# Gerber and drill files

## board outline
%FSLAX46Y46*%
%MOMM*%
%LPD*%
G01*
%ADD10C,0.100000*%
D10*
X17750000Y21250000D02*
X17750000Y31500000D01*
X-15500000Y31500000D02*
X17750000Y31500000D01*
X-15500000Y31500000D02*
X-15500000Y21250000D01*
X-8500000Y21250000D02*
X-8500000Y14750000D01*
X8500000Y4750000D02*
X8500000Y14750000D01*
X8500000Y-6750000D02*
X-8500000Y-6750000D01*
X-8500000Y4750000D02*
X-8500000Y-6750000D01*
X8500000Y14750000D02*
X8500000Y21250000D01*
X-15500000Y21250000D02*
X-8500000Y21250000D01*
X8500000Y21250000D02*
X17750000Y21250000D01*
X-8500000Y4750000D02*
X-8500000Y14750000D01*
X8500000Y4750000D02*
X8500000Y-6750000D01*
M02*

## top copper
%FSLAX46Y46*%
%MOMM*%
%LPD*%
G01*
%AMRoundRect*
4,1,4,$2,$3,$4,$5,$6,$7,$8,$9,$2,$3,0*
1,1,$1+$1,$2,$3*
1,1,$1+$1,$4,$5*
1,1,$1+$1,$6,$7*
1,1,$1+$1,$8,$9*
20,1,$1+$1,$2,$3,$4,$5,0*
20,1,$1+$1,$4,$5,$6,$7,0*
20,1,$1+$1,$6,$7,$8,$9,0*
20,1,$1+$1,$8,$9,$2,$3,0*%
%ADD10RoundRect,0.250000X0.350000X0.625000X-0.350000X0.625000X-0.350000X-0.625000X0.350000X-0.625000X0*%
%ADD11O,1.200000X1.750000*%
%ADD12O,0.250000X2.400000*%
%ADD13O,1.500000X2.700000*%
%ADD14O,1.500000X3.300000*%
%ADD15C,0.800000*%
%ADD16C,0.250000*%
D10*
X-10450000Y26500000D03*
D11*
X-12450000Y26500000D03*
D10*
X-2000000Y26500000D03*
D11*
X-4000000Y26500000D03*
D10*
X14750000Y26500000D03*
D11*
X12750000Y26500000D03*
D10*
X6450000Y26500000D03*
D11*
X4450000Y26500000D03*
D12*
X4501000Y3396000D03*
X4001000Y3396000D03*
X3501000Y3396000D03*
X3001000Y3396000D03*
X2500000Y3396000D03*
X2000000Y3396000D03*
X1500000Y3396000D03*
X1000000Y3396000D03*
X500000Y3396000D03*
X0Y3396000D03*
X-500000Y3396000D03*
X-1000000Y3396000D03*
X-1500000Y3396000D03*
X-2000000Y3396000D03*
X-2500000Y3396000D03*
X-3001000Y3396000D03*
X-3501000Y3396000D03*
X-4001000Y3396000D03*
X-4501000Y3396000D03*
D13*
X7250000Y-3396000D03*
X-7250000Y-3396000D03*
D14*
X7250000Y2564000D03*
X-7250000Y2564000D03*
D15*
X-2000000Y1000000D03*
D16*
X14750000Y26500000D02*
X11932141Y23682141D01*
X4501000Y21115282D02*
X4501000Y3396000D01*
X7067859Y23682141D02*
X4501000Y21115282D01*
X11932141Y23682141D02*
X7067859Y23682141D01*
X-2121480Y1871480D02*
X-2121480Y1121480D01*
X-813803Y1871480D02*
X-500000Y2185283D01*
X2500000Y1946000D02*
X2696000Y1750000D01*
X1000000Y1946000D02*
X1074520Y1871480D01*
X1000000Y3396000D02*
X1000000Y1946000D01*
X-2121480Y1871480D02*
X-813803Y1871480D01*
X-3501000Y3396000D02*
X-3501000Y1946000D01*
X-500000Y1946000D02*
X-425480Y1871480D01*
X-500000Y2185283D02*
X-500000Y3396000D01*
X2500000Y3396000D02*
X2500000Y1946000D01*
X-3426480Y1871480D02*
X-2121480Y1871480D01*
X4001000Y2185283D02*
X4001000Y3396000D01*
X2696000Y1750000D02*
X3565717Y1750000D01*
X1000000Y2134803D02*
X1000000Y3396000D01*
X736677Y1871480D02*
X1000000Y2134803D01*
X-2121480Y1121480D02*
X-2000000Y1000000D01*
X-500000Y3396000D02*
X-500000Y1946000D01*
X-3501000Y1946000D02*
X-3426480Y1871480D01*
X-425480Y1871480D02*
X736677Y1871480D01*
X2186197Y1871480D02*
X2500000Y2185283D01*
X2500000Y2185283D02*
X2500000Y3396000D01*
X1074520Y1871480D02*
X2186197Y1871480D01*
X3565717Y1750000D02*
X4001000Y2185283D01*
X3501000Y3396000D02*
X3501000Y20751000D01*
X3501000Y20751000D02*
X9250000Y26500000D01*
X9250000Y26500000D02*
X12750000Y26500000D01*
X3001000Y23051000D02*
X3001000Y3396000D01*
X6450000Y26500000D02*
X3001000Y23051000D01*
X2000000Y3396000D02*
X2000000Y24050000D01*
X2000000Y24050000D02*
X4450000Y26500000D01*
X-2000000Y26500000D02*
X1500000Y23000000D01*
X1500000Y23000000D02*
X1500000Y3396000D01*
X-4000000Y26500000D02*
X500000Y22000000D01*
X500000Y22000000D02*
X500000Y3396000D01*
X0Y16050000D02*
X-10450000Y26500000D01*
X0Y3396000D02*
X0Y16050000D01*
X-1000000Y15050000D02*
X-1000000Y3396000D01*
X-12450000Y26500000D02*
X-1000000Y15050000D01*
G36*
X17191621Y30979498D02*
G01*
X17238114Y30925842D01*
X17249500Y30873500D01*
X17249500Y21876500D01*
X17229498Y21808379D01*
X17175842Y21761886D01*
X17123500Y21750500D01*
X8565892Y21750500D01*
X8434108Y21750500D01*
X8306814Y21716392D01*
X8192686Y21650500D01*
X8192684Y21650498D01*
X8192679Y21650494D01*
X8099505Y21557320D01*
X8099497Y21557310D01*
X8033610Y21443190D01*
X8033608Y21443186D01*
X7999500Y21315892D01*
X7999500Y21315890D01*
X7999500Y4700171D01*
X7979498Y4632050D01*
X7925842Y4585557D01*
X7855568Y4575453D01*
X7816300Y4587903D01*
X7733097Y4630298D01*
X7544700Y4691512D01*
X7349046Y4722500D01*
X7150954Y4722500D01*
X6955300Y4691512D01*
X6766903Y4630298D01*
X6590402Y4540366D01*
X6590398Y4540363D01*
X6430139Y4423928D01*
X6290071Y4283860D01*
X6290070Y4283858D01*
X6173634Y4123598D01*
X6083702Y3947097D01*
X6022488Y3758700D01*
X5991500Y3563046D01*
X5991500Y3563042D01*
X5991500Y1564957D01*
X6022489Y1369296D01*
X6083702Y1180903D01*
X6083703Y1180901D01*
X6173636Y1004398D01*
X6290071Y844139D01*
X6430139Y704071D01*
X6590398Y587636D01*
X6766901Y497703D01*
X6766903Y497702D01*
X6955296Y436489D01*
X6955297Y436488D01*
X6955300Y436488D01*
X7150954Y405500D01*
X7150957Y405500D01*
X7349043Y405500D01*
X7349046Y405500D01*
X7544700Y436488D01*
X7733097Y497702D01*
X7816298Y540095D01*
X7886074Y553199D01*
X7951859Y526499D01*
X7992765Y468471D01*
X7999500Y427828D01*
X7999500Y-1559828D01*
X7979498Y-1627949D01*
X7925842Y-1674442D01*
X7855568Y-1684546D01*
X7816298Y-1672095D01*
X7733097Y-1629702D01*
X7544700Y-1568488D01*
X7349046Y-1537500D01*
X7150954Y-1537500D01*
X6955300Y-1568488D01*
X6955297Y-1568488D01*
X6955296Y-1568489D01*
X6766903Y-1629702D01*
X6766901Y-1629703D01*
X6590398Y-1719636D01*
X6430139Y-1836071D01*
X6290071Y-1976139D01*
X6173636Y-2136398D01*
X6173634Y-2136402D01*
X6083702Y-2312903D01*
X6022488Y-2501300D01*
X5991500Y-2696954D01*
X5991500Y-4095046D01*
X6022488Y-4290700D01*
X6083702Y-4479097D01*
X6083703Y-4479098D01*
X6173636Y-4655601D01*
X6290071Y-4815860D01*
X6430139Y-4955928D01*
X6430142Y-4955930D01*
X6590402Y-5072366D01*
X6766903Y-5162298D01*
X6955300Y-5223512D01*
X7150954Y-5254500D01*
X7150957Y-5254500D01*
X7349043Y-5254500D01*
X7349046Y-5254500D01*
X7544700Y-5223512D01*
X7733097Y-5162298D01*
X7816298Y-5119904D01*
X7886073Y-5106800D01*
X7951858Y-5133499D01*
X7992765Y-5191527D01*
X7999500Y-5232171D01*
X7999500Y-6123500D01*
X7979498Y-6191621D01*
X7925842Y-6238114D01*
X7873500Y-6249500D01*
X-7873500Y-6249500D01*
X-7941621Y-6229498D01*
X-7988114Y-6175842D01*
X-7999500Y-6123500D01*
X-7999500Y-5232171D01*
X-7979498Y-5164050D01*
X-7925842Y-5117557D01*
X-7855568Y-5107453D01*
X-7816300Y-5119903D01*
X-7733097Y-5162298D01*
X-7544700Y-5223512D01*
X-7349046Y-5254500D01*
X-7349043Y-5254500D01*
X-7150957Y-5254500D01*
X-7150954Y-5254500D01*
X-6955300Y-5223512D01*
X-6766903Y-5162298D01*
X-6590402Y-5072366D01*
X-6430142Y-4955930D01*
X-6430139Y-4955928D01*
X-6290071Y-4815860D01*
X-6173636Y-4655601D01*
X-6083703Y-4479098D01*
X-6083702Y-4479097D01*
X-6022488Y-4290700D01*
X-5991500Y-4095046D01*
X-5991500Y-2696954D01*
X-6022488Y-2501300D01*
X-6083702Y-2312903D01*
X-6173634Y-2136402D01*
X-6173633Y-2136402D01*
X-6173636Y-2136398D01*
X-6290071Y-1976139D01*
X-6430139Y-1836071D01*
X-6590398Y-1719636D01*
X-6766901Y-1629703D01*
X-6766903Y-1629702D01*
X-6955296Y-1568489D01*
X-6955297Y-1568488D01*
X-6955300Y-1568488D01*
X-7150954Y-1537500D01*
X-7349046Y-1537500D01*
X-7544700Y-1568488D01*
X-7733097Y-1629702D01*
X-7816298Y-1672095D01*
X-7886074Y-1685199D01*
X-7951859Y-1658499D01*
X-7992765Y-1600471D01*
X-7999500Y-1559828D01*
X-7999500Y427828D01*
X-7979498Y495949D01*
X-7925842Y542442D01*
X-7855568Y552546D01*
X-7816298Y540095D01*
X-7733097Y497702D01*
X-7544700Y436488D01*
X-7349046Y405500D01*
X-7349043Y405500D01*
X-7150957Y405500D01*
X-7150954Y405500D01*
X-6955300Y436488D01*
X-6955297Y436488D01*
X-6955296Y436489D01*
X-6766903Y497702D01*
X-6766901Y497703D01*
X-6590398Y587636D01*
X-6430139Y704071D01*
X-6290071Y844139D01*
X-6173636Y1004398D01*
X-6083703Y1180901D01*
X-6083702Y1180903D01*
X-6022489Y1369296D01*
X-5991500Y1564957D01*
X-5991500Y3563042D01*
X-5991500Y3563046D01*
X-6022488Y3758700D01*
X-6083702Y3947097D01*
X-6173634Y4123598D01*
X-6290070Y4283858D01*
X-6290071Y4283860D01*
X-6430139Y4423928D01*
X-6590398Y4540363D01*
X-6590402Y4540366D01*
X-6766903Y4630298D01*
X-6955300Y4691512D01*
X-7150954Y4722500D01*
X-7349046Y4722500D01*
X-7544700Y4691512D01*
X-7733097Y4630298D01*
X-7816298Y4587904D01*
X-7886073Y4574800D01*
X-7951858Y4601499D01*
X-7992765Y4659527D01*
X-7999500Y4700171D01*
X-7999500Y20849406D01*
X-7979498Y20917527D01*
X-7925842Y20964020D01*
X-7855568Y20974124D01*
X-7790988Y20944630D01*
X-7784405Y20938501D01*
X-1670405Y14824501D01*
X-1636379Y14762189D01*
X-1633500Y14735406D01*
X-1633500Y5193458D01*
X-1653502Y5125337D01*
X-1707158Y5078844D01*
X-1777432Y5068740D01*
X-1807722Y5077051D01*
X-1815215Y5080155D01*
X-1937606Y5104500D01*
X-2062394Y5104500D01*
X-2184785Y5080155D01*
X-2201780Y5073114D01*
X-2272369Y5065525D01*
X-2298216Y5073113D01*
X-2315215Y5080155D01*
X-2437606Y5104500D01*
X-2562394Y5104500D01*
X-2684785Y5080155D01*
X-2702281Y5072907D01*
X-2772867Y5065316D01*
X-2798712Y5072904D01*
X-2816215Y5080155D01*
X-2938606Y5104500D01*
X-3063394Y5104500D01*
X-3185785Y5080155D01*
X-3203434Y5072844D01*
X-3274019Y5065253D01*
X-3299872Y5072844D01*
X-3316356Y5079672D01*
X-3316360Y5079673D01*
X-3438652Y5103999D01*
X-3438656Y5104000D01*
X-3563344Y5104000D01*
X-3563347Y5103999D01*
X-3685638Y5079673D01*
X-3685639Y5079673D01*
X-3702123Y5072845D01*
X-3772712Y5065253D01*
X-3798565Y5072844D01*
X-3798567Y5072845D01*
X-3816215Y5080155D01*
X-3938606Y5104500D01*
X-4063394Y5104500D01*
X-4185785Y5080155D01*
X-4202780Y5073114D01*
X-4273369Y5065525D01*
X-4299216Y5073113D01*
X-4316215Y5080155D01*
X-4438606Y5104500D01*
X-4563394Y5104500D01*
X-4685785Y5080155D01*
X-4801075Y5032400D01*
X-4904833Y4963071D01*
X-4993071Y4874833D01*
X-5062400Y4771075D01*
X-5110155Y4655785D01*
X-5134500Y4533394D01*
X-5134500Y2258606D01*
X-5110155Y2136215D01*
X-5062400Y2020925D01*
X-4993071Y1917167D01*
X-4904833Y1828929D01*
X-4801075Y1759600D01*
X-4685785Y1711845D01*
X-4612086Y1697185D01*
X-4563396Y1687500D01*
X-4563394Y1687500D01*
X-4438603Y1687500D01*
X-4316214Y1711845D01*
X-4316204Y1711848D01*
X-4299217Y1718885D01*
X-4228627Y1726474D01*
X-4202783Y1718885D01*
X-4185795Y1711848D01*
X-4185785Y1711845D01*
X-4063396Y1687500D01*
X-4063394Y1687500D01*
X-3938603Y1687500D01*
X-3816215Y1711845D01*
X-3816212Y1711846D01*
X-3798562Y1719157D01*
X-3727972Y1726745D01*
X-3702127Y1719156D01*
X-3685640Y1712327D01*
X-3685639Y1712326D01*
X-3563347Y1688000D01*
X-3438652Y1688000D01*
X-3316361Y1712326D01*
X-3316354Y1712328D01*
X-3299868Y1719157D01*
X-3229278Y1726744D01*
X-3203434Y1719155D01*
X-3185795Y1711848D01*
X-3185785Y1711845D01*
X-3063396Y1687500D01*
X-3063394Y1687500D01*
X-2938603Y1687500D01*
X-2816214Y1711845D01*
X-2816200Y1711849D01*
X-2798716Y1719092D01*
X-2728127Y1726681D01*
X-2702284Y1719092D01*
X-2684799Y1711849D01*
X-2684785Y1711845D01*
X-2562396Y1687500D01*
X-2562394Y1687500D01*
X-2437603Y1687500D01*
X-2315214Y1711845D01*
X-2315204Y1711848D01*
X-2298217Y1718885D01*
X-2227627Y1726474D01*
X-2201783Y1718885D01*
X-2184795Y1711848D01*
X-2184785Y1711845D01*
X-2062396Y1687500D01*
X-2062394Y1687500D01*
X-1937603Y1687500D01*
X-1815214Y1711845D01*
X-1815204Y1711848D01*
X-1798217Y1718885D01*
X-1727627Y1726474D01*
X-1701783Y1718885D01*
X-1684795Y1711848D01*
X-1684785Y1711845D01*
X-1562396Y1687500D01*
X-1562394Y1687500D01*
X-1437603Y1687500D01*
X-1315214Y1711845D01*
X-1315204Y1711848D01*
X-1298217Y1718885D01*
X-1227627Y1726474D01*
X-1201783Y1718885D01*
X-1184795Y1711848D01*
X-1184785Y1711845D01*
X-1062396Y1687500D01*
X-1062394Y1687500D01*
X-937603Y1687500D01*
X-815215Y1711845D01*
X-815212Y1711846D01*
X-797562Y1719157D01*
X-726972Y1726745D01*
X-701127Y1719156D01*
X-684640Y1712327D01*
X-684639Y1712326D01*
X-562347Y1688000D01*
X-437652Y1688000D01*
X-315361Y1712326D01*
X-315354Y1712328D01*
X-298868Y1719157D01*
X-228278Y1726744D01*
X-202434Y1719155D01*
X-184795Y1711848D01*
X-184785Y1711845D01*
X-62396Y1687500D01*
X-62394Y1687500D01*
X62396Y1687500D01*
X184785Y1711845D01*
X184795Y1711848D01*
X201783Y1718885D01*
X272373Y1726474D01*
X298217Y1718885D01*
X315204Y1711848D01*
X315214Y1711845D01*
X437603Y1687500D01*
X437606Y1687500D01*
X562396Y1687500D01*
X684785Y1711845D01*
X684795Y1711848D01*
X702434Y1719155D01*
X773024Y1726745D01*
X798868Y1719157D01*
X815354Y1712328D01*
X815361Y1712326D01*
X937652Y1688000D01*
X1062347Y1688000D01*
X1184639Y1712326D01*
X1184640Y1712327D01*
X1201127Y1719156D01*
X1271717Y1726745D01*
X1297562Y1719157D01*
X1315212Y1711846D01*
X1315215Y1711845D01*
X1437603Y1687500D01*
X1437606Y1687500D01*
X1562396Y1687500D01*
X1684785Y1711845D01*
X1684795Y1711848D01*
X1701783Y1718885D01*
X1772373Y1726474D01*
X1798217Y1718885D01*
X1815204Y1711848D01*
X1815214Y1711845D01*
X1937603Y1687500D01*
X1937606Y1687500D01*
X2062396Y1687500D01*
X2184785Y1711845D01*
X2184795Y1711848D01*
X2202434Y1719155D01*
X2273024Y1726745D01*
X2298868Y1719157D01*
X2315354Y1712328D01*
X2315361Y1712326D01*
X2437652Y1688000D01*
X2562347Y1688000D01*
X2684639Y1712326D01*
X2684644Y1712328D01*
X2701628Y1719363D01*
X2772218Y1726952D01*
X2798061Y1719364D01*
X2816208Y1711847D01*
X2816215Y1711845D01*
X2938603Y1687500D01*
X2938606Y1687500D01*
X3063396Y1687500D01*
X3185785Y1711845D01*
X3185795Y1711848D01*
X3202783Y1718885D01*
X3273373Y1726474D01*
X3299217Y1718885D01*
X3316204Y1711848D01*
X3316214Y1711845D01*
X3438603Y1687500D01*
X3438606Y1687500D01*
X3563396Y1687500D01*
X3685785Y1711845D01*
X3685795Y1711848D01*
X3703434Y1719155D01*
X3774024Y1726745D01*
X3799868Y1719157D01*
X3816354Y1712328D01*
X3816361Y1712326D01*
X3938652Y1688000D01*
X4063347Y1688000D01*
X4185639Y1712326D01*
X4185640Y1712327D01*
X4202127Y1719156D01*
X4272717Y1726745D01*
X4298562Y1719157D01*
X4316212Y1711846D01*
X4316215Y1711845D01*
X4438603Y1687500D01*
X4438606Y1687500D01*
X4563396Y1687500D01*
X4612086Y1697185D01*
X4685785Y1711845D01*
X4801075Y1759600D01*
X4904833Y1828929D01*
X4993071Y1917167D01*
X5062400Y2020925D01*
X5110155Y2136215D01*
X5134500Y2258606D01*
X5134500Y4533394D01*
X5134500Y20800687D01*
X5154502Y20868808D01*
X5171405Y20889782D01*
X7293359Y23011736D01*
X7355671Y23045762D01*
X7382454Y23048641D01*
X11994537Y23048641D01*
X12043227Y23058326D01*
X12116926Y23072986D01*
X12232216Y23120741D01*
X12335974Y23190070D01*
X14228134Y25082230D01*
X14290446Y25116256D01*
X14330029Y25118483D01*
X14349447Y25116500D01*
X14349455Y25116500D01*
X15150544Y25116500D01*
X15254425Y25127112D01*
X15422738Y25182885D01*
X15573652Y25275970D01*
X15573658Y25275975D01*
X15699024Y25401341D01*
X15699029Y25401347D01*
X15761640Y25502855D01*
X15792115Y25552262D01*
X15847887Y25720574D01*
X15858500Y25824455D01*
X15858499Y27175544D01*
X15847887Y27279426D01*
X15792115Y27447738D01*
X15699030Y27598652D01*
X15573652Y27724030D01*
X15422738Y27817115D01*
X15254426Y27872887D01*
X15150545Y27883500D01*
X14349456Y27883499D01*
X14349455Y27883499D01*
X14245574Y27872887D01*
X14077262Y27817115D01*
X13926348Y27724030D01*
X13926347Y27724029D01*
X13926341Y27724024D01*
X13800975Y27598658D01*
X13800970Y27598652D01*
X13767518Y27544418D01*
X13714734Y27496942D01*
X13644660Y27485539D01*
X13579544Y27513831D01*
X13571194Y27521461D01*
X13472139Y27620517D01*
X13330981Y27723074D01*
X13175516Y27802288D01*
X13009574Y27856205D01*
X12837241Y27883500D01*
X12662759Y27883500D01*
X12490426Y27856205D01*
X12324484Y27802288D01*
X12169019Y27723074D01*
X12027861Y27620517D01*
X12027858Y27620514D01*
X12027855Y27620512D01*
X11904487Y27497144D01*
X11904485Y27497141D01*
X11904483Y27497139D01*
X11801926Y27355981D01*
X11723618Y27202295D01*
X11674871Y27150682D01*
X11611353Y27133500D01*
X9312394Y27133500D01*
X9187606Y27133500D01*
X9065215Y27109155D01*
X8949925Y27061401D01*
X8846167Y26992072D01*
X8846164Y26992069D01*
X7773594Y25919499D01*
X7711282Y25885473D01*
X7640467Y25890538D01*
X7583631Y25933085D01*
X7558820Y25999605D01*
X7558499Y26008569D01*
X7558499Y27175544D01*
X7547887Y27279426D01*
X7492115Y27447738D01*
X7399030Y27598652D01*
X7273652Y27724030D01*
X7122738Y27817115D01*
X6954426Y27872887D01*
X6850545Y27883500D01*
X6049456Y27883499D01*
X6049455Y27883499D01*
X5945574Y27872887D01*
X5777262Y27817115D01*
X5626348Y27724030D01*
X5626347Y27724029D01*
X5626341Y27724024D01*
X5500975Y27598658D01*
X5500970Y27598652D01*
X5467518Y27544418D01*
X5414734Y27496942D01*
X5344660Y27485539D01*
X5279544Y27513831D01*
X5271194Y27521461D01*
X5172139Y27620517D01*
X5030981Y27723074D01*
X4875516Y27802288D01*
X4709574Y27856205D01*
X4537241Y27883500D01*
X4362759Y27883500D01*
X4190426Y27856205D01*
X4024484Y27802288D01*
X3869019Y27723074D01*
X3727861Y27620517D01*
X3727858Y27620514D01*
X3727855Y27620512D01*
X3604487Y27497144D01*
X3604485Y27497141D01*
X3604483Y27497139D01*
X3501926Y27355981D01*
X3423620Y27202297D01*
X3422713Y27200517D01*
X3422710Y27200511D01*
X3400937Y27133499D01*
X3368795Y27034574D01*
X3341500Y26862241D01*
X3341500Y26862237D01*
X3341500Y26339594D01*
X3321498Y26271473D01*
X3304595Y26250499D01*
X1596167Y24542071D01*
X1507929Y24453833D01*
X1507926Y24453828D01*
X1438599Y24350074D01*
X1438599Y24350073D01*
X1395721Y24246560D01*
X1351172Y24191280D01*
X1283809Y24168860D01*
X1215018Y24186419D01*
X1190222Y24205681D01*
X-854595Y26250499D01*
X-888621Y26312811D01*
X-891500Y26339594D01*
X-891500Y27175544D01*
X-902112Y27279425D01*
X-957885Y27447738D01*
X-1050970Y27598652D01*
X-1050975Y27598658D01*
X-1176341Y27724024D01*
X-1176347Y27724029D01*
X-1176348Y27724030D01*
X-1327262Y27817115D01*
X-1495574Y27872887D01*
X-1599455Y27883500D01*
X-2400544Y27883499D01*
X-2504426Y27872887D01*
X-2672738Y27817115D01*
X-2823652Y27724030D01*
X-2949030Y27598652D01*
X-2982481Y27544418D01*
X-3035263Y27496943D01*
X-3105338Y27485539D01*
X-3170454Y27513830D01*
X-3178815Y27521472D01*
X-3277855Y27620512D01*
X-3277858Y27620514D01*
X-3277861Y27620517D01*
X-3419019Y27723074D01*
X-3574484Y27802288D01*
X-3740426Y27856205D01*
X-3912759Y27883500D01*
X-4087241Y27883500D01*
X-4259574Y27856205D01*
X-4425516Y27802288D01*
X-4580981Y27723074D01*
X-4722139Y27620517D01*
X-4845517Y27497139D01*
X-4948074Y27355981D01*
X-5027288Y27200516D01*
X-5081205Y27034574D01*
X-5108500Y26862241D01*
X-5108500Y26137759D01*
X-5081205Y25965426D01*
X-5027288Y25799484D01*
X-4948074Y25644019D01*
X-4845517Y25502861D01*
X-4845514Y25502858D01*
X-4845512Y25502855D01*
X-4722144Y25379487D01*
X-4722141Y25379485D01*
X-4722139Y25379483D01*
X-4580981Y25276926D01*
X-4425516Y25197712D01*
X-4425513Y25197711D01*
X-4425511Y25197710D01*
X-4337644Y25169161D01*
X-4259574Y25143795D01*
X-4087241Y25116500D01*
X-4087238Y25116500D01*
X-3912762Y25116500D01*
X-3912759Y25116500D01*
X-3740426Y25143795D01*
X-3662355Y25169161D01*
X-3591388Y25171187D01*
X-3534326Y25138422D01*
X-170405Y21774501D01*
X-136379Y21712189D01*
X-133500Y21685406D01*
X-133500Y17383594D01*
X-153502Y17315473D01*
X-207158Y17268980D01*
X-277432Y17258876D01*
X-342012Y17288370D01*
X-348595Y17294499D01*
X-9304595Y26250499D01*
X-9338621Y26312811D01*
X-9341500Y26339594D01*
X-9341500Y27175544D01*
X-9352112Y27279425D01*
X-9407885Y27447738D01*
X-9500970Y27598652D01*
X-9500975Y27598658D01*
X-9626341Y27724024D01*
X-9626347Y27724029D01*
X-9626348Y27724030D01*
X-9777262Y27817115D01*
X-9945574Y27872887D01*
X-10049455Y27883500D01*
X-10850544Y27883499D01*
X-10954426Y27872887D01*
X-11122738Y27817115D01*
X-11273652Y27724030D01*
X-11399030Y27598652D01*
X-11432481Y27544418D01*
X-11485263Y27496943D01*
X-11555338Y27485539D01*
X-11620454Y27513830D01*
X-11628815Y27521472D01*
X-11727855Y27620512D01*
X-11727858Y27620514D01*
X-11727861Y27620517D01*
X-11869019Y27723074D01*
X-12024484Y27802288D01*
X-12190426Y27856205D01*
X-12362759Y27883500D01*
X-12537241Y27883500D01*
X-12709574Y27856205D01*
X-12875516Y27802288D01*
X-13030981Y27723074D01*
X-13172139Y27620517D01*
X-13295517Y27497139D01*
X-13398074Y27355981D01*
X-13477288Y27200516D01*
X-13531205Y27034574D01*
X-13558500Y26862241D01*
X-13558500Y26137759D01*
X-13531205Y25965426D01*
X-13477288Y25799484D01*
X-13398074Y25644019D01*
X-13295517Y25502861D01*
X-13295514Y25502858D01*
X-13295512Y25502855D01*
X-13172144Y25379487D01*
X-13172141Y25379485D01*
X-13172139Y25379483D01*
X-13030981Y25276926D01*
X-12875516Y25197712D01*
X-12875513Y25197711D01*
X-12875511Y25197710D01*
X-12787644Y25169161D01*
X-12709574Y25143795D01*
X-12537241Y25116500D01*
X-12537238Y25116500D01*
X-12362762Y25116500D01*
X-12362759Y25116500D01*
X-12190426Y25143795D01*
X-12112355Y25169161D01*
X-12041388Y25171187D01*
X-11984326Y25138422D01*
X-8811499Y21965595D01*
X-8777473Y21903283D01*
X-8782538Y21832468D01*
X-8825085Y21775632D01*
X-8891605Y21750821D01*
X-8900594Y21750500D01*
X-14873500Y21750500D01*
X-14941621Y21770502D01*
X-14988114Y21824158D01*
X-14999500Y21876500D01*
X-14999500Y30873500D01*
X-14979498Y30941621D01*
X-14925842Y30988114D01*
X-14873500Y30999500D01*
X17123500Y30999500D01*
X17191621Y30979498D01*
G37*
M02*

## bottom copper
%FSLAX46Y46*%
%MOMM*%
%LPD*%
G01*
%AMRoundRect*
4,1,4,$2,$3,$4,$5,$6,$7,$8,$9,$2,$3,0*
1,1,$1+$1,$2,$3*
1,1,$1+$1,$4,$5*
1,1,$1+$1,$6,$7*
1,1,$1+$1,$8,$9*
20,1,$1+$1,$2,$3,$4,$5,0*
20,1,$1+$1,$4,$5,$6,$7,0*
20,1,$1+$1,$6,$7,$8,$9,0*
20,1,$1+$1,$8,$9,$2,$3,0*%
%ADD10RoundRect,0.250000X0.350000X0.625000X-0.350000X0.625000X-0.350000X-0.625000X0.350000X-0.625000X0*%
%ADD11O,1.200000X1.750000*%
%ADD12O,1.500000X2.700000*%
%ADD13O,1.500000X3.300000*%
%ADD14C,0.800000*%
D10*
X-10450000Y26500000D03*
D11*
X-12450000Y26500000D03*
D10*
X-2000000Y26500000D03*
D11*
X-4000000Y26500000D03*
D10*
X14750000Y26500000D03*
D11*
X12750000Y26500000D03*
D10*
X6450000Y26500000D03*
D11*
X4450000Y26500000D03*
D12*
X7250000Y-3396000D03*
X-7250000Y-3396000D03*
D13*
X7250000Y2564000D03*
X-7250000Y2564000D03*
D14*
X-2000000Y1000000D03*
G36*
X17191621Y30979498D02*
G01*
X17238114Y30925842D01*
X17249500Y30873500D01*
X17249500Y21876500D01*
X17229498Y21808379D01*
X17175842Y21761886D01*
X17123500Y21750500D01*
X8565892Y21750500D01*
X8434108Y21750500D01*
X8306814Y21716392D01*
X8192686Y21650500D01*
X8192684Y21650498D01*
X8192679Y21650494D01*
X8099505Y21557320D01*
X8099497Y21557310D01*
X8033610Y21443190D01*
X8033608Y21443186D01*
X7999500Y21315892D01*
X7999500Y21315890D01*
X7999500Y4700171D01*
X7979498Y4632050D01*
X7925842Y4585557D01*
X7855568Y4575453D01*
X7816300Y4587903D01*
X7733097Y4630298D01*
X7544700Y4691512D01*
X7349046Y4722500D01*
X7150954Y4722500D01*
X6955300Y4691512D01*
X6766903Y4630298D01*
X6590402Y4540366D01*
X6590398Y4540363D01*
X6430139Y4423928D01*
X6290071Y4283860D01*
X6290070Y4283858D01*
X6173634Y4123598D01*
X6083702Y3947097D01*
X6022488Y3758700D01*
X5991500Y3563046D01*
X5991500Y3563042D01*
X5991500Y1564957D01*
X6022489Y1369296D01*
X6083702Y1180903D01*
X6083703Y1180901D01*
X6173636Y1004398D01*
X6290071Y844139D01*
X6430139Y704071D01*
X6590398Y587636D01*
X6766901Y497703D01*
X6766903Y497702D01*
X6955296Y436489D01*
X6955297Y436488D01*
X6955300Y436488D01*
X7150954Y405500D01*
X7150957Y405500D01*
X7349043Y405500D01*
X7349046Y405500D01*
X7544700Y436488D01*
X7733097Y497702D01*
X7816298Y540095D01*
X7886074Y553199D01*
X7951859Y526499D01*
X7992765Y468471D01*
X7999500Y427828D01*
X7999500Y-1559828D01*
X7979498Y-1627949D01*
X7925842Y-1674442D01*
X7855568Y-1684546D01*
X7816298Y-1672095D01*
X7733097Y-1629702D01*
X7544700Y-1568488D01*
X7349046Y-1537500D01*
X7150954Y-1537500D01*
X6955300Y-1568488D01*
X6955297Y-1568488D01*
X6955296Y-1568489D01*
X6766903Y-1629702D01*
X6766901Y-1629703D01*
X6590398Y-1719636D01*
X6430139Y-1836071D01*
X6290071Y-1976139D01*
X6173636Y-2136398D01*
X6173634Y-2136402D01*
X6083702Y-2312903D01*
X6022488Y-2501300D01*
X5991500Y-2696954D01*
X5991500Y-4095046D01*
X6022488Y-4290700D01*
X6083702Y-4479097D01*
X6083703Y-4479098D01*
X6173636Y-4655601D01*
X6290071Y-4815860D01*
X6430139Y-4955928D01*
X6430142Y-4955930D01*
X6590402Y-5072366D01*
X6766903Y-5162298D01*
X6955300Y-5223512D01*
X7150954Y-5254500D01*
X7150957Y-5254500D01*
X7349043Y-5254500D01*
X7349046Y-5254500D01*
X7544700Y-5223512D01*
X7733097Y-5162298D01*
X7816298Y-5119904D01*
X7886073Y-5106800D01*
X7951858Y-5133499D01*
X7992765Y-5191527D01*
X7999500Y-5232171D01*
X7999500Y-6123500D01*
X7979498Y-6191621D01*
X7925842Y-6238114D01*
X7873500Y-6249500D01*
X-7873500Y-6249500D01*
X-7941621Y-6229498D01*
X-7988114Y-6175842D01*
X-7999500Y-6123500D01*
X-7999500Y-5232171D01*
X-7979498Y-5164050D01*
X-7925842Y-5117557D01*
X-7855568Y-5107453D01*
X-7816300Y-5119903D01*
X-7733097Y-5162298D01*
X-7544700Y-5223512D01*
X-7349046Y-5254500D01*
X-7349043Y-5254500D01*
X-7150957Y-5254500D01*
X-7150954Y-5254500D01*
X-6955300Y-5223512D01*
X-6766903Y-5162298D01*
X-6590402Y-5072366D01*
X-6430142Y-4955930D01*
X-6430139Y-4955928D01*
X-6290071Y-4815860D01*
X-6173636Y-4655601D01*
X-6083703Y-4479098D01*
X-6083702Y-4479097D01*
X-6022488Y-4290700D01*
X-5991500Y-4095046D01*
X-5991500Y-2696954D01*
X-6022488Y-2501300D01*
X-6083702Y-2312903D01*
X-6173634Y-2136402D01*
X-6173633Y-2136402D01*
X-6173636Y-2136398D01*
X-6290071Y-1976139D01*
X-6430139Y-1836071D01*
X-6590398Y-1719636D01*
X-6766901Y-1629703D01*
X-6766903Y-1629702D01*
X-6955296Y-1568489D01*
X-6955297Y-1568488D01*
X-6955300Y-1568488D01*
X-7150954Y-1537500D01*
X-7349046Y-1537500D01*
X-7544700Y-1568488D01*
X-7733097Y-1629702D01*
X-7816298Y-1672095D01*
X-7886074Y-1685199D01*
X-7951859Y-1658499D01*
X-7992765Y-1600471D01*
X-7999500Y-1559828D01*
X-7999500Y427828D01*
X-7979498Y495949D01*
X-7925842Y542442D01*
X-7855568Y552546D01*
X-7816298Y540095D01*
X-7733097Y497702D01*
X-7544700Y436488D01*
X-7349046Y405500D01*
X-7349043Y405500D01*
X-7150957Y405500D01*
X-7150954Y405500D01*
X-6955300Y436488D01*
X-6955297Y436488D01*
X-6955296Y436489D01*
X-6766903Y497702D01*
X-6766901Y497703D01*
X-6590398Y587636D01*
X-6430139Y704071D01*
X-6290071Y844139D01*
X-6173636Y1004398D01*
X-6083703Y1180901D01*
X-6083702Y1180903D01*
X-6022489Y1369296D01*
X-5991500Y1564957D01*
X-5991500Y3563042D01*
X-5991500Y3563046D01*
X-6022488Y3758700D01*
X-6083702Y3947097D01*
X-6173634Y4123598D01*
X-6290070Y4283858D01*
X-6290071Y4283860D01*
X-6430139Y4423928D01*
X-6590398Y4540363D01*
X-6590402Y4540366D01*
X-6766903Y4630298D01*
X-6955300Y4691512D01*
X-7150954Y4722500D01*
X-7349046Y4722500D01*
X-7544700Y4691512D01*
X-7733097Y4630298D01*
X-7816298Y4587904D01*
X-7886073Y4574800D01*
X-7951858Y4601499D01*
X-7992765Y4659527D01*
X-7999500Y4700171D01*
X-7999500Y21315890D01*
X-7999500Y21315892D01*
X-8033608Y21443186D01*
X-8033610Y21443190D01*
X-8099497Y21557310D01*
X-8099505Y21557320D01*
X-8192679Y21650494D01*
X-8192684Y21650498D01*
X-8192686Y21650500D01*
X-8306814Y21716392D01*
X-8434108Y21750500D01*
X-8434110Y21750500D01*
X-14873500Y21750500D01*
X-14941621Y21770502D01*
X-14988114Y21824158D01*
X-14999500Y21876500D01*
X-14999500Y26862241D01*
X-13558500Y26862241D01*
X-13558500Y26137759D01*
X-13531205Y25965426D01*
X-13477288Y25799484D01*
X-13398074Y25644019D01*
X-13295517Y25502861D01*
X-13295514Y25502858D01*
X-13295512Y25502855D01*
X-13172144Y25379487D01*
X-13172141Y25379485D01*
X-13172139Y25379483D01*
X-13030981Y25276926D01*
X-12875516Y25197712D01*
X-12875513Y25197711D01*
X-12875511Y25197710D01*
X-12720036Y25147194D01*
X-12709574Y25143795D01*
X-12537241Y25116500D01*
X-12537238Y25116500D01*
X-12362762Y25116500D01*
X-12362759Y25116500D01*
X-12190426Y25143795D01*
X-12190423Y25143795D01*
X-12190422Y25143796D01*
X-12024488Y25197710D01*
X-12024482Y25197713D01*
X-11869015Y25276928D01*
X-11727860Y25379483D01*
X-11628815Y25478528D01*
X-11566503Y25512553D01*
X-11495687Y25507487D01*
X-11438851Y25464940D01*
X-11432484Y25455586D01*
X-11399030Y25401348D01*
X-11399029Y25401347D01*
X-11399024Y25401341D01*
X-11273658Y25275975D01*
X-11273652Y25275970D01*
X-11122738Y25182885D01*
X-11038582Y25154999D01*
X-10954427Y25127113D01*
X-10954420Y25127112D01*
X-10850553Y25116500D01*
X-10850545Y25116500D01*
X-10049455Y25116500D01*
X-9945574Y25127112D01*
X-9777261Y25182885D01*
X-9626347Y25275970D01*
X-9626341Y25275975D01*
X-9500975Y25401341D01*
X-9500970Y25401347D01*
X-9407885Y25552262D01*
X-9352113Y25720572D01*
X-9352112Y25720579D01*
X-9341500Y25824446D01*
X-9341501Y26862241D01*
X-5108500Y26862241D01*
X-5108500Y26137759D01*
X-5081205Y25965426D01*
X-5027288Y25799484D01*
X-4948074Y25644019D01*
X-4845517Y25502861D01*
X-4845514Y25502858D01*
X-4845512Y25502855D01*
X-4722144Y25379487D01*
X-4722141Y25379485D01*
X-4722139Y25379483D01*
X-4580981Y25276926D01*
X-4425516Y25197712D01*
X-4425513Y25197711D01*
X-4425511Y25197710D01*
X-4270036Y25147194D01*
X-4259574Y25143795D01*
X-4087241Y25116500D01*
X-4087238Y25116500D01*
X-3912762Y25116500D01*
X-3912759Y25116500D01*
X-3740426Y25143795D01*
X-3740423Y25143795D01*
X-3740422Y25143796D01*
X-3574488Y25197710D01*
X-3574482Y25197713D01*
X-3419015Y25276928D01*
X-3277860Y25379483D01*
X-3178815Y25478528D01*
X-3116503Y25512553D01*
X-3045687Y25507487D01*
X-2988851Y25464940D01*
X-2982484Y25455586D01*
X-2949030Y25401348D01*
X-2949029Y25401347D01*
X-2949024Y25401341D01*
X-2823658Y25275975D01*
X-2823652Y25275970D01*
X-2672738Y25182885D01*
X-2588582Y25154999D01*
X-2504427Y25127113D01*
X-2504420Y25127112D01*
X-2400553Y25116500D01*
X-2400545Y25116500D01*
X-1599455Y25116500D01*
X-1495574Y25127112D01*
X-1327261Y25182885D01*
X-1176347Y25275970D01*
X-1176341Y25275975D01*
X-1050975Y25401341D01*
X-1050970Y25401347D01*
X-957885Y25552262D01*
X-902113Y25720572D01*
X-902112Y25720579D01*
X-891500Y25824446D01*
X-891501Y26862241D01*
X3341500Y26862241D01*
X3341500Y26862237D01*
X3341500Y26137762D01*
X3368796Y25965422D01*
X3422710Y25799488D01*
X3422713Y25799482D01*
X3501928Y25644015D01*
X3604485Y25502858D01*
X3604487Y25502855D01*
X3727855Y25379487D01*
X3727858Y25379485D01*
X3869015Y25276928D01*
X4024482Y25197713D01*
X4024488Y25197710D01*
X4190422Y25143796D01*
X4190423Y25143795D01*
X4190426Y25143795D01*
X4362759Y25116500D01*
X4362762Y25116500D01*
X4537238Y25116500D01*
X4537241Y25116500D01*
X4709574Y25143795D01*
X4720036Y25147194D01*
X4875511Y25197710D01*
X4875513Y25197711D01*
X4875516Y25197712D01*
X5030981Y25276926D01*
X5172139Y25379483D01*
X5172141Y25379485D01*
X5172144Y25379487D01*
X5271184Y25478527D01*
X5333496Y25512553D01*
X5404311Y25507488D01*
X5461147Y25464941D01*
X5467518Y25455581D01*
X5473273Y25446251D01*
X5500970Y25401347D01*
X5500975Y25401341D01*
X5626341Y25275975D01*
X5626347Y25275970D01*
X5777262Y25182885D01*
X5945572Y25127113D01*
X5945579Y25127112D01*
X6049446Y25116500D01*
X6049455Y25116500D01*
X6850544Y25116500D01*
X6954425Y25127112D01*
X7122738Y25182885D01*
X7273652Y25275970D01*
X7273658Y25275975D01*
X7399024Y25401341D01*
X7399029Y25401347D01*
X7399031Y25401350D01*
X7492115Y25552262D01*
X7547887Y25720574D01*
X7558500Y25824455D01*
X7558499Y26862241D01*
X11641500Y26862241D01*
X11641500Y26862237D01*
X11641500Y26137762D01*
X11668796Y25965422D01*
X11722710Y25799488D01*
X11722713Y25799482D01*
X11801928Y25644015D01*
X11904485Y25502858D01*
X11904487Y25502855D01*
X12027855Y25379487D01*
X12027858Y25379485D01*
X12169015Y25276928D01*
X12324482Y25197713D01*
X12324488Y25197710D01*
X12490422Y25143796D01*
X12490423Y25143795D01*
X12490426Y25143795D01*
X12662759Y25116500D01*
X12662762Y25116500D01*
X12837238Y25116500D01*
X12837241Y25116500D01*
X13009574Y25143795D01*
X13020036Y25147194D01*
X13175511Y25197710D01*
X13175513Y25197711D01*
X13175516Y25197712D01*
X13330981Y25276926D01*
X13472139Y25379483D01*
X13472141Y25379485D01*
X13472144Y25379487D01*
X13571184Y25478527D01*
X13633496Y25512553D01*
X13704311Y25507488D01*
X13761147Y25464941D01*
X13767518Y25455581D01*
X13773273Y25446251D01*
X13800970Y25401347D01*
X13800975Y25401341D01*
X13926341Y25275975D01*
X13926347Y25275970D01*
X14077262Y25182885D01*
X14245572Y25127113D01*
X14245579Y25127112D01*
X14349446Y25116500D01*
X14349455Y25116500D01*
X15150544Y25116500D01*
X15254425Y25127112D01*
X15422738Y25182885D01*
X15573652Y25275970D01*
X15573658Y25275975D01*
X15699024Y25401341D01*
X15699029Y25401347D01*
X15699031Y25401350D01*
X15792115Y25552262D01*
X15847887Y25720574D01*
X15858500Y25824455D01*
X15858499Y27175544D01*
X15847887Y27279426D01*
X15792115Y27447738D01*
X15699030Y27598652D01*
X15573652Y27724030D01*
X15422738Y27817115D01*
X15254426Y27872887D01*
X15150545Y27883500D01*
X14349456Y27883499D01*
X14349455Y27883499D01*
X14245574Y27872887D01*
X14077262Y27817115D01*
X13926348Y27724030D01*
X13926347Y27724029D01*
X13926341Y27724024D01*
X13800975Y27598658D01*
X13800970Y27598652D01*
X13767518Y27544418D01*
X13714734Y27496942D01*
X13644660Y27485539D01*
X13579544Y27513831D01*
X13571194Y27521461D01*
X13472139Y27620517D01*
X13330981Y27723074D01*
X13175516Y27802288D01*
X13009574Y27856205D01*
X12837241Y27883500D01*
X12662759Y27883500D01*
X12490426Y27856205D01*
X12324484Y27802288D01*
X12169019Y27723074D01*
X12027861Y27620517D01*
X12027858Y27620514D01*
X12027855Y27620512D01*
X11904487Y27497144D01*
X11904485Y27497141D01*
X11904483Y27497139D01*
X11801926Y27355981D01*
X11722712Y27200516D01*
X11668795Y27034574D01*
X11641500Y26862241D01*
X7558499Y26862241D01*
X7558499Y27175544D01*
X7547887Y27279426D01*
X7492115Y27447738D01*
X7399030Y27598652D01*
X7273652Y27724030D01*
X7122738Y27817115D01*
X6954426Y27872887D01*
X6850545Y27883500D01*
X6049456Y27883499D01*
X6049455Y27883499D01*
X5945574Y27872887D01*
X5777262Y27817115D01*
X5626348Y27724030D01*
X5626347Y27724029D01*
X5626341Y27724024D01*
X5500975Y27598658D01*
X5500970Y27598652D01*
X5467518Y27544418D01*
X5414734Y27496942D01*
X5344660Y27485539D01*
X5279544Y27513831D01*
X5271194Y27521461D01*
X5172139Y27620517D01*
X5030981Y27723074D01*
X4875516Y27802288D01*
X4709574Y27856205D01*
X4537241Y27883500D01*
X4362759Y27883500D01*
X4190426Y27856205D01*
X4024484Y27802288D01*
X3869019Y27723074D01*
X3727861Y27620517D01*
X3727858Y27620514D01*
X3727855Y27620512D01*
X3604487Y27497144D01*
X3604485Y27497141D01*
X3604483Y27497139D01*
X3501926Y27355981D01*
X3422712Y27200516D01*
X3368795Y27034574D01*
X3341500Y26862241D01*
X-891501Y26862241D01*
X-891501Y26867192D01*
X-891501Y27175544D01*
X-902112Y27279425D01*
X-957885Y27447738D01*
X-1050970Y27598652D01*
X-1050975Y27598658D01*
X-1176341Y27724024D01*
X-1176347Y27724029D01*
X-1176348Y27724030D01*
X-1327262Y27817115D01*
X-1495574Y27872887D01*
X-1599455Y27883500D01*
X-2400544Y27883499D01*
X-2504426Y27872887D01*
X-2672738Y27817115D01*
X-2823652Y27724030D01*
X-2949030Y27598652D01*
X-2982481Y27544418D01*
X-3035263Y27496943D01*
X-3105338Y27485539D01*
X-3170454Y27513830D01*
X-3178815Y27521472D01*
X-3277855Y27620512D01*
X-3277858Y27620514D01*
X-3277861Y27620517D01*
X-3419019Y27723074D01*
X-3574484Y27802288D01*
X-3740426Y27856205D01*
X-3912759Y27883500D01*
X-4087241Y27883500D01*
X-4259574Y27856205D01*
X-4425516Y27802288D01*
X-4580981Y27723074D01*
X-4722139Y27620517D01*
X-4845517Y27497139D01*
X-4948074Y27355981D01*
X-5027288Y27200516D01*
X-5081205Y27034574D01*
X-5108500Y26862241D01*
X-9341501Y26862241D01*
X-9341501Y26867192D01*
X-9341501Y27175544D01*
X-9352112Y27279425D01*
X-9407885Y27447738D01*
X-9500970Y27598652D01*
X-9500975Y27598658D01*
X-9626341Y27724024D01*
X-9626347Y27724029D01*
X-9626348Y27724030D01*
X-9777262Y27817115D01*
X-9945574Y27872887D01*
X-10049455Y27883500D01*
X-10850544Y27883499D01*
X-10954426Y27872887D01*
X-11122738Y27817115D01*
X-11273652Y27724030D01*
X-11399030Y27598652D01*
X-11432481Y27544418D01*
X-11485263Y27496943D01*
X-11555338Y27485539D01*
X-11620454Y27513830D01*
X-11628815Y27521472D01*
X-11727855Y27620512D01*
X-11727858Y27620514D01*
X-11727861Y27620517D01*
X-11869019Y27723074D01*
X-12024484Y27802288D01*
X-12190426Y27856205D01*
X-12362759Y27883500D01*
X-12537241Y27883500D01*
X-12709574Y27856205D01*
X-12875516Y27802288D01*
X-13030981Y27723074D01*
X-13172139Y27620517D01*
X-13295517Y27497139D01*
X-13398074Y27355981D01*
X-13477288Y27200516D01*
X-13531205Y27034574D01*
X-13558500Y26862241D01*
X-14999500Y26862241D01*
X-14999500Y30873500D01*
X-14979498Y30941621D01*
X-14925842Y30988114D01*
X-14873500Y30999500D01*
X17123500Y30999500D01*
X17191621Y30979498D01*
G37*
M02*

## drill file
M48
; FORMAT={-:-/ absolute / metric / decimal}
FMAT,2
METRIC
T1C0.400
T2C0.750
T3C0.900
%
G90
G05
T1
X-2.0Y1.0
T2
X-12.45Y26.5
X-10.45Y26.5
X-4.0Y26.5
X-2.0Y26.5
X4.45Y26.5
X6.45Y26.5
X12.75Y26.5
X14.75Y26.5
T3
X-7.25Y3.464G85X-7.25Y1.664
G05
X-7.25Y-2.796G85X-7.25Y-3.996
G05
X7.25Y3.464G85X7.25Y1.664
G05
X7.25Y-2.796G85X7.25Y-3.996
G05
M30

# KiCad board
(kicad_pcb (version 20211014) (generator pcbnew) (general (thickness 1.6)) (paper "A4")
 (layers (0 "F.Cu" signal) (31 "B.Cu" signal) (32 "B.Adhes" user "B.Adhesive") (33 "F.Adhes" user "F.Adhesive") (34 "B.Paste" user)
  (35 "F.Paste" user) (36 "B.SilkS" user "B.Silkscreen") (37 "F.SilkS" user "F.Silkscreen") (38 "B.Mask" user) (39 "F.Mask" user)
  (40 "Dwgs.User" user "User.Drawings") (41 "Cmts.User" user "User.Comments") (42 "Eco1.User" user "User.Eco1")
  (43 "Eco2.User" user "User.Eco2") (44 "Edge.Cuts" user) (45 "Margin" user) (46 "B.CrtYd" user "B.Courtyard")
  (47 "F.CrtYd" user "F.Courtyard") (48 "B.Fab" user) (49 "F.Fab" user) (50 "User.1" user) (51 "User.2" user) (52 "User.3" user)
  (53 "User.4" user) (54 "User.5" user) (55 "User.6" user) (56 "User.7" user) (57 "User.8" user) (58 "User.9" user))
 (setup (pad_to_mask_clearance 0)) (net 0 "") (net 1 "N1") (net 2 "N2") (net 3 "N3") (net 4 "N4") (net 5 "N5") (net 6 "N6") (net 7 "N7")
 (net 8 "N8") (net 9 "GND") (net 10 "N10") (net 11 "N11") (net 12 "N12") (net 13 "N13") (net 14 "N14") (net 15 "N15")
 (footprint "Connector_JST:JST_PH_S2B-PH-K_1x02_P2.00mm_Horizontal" (layer "F.Cu") (at -10.45 -26.5 180)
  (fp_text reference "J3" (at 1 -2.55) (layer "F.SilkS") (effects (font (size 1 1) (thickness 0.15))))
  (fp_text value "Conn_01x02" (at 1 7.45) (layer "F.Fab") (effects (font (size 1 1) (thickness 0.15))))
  (pad "1" thru_hole roundrect (at 0 0 180) (size 1.2 1.75) (drill 0.75) (layers *.Cu *.Mask) (roundrect_rratio 0.2083333333) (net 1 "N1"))
  (pad "2" thru_hole oval (at 2 0 180) (size 1.2 1.75) (drill 0.75) (layers *.Cu *.Mask) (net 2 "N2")))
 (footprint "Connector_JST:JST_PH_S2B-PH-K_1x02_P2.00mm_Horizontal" (layer "F.Cu") (at -2 -26.5 180)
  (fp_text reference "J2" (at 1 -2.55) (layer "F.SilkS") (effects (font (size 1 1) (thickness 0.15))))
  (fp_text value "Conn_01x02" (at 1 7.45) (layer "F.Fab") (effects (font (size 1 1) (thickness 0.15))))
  (pad "1" thru_hole roundrect (at 0 0 180) (size 1.2 1.75) (drill 0.75) (layers *.Cu *.Mask) (roundrect_rratio 0.2083333333) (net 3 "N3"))
  (pad "2" thru_hole oval (at 2 0 180) (size 1.2 1.75) (drill 0.75) (layers *.Cu *.Mask) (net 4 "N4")))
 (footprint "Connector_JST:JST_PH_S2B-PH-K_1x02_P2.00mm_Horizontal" (layer "F.Cu") (at 14.75 -26.5 180)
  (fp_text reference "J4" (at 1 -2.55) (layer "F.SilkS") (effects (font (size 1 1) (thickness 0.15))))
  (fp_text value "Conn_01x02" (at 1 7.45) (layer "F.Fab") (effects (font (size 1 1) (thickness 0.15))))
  (pad "1" thru_hole roundrect (at 0 0 180) (size 1.2 1.75) (drill 0.75) (layers *.Cu *.Mask) (roundrect_rratio 0.2083333333) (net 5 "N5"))
  (pad "2" thru_hole oval (at 2 0 180) (size 1.2 1.75) (drill 0.75) (layers *.Cu *.Mask) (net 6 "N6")))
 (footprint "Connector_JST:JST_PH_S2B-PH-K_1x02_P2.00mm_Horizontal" (layer "F.Cu") (at 6.45 -26.5 180)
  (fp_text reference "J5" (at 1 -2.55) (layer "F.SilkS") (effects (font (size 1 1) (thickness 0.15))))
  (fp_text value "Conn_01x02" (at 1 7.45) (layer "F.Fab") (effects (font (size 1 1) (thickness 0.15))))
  (pad "1" thru_hole roundrect (at 0 0 180) (size 1.2 1.75) (drill 0.75) (layers *.Cu *.Mask) (roundrect_rratio 0.2083333333) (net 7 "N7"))
  (pad "2" thru_hole oval (at 2 0 180) (size 1.2 1.75) (drill 0.75) (layers *.Cu *.Mask) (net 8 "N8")))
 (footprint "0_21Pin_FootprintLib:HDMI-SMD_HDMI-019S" (layer "F.Cu") (at 0 0)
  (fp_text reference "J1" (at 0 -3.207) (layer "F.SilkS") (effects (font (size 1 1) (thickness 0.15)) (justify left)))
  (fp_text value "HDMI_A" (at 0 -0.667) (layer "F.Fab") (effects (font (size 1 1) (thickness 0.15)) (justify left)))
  (pad "1" smd oval (at 4.501 -3.396) (size 0.25 2.4) (layers "F.Cu" "F.Paste" "F.Mask") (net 5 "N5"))
  (pad "2" smd oval (at 4.001 -3.396) (size 0.25 2.4) (layers "F.Cu" "F.Paste" "F.Mask") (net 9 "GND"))
  (pad "3" smd oval (at 3.501 -3.396) (size 0.25 2.4) (layers "F.Cu" "F.Paste" "F.Mask") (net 6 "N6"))
  (pad "4" smd oval (at 3.001 -3.396) (size 0.25 2.4) (layers "F.Cu" "F.Paste" "F.Mask") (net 7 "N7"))
  (pad "5" smd oval (at 2.5 -3.396) (size 0.25 2.4) (layers "F.Cu" "F.Paste" "F.Mask") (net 9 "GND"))
  (pad "6" smd oval (at 2 -3.396) (size 0.25 2.4) (layers "F.Cu" "F.Paste" "F.Mask") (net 8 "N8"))
  (pad "7" smd oval (at 1.5 -3.396) (size 0.25 2.4) (layers "F.Cu" "F.Paste" "F.Mask") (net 3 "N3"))
  (pad "8" smd oval (at 1 -3.396) (size 0.25 2.4) (layers "F.Cu" "F.Paste" "F.Mask") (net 9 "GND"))
  (pad "9" smd oval (at 0.5 -3.396) (size 0.25 2.4) (layers "F.Cu" "F.Paste" "F.Mask") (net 4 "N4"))
  (pad "10" smd oval (at 0 -3.396) (size 0.25 2.4) (layers "F.Cu" "F.Paste" "F.Mask") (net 1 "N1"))
  (pad "11" smd oval (at -0.5 -3.396) (size 0.25 2.4) (layers "F.Cu" "F.Paste" "F.Mask") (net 9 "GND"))
  (pad "12" smd oval (at -1 -3.396) (size 0.25 2.4) (layers "F.Cu" "F.Paste" "F.Mask") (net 2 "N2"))
  (pad "13" smd oval (at -1.5 -3.396) (size 0.25 2.4) (layers "F.Cu" "F.Paste" "F.Mask") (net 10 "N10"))
  (pad "14" smd oval (at -2 -3.396) (size 0.25 2.4) (layers "F.Cu" "F.Paste" "F.Mask") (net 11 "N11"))
  (pad "15" smd oval (at -2.5 -3.396) (size 0.25 2.4) (layers "F.Cu" "F.Paste" "F.Mask") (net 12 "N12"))
  (pad "16" smd oval (at -3.001 -3.396) (size 0.25 2.4) (layers "F.Cu" "F.Paste" "F.Mask") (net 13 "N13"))
  (pad "17" smd oval (at -3.501 -3.396) (size 0.25 2.4) (layers "F.Cu" "F.Paste" "F.Mask") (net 9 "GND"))
  (pad "18" smd oval (at -4.001 -3.396) (size 0.25 2.4) (layers "F.Cu" "F.Paste" "F.Mask") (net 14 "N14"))
  (pad "19" smd oval (at -4.501 -3.396) (size 0.25 2.4) (layers "F.Cu" "F.Paste" "F.Mask") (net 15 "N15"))
  (pad "20" thru_hole oval (at 7.25 3.396) (size 1.5 2.7) (drill oval 0.9 2.1) (layers *.Cu *.Mask))
  (pad "21" thru_hole oval (at -7.25 3.396) (size 1.5 2.7) (drill oval 0.9 2.1) (layers *.Cu *.Mask))
  (pad "22" thru_hole oval (at 7.25 -2.564) (size 1.5 3.3) (drill oval 0.9 2.7) (layers *.Cu *.Mask))
  (pad "23" thru_hole oval (at -7.25 -2.564) (size 1.5 3.3) (drill oval 0.9 2.7) (layers *.Cu *.Mask)))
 (gr_line (start 17.75 -21.25) (end 17.75 -31.5) (layer "Edge.Cuts") (width 0.1))
 (gr_line (start -15.5 -31.5) (end 17.75 -31.5) (layer "Edge.Cuts") (width 0.1))
 (gr_line (start -15.5 -31.5) (end -15.5 -21.25) (layer "Edge.Cuts") (width 0.1))
 (gr_line (start -8.5 -21.25) (end -8.5 -14.75) (layer "Edge.Cuts") (width 0.1))
 (gr_line (start 8.5 -4.75) (end 8.5 -14.75) (layer "Edge.Cuts") (width 0.1))
 (gr_line (start 8.5 6.75) (end -8.5 6.75) (layer "Edge.Cuts") (width 0.1))
 (gr_line (start -8.5 -4.75) (end -8.5 6.75) (layer "Edge.Cuts") (width 0.1))
 (gr_line (start 8.5 -14.75) (end 8.5 -21.25) (layer "Edge.Cuts") (width 0.1))
 (gr_line (start -15.5 -21.25) (end -8.5 -21.25) (layer "Edge.Cuts") (width 0.1))
 (gr_line (start 8.5 -21.25) (end 17.75 -21.25) (layer "Edge.Cuts") (width 0.1))
 (gr_line (start -8.5 -4.75) (end -8.5 -14.75) (layer "Edge.Cuts") (width 0.1))
 (gr_line (start 8.5 -4.75) (end 8.5 6.75) (layer "Edge.Cuts") (width 0.1))
 (segment (start 14.75 -26.5) (end 11.932141 -23.682141) (width 0.25) (layer "F.Cu") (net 5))
 (segment (start 4.501 -21.115282) (end 4.501 -3.396) (width 0.25) (layer "F.Cu") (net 5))
 (segment (start 7.067859 -23.682141) (end 4.501 -21.115282) (width 0.25) (layer "F.Cu") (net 5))
 (segment (start 11.932141 -23.682141) (end 7.067859 -23.682141) (width 0.25) (layer "F.Cu") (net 5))
 (segment (start -2.12148 -1.87148) (end -2.12148 -1.12148) (width 0.25) (layer "F.Cu") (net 9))
 (segment (start -0.813803 -1.87148) (end -0.5 -2.185283) (width 0.25) (layer "F.Cu") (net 9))
 (segment (start 2.5 -1.946) (end 2.696 -1.75) (width 0.25) (layer "F.Cu") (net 9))
 (segment (start 1 -1.946) (end 1.07452 -1.87148) (width 0.25) (layer "F.Cu") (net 9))
 (segment (start 1 -3.396) (end 1 -1.946) (width 0.25) (layer "F.Cu") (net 9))
 (segment (start -2.12148 -1.87148) (end -0.813803 -1.87148) (width 0.25) (layer "F.Cu") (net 9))
 (segment (start -3.501 -3.396) (end -3.501 -1.946) (width 0.25) (layer "F.Cu") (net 9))
 (segment (start -0.5 -1.946) (end -0.42548 -1.87148) (width 0.25) (layer "F.Cu") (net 9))
 (segment (start -0.5 -2.185283) (end -0.5 -3.396) (width 0.25) (layer "F.Cu") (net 9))
 (segment (start 2.5 -3.396) (end 2.5 -1.946) (width 0.25) (layer "F.Cu") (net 9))
 (segment (start -3.42648 -1.87148) (end -2.12148 -1.87148) (width 0.25) (layer "F.Cu") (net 9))
 (segment (start 4.001 -2.185283) (end 4.001 -3.396) (width 0.25) (layer "F.Cu") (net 9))
 (segment (start 2.696 -1.75) (end 3.565717 -1.75) (width 0.25) (layer "F.Cu") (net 9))
 (segment (start 1 -2.134803) (end 1 -3.396) (width 0.25) (layer "F.Cu") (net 9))
 (segment (start 0.736677 -1.87148) (end 1 -2.134803) (width 0.25) (layer "F.Cu") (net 9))
 (segment (start -2.12148 -1.12148) (end -2 -1) (width 0.25) (layer "F.Cu") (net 9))
 (segment (start -0.5 -3.396) (end -0.5 -1.946) (width 0.25) (layer "F.Cu") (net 9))
 (segment (start -3.501 -1.946) (end -3.42648 -1.87148) (width 0.25) (layer "F.Cu") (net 9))
 (segment (start -0.42548 -1.87148) (end 0.736677 -1.87148) (width 0.25) (layer "F.Cu") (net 9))
 (segment (start 2.186197 -1.87148) (end 2.5 -2.185283) (width 0.25) (layer "F.Cu") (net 9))
 (segment (start 2.5 -2.185283) (end 2.5 -3.396) (width 0.25) (layer "F.Cu") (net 9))
 (segment (start 1.07452 -1.87148) (end 2.186197 -1.87148) (width 0.25) (layer "F.Cu") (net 9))
 (segment (start 3.565717 -1.75) (end 4.001 -2.185283) (width 0.25) (layer "F.Cu") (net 9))
 (via (at -2 -1) (size 0.8) (drill 0.4) (layers "F.Cu" "B.Cu") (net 9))
 (segment (start 3.501 -3.396) (end 3.501 -20.751) (width 0.25) (layer "F.Cu") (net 6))
 (segment (start 3.501 -20.751) (end 9.25 -26.5) (width 0.25) (layer "F.Cu") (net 6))
 (segment (start 9.25 -26.5) (end 12.75 -26.5) (width 0.25) (layer "F.Cu") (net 6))
 (segment (start 3.001 -23.051) (end 3.001 -3.396) (width 0.25) (layer "F.Cu") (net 7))
 (segment (start 6.45 -26.5) (end 3.001 -23.051) (width 0.25) (layer "F.Cu") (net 7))
 (segment (start 2 -3.396) (end 2 -24.05) (width 0.25) (layer "F.Cu") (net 8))
 (segment (start 2 -24.05) (end 4.45 -26.5) (width 0.25) (layer "F.Cu") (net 8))
 (segment (start -2 -26.5) (end 1.5 -23) (width 0.25) (layer "F.Cu") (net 3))
 (segment (start 1.5 -23) (end 1.5 -3.396) (width 0.25) (layer "F.Cu") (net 3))
 (segment (start -4 -26.5) (end 0.5 -22) (width 0.25) (layer "F.Cu") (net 4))
 (segment (start 0.5 -22) (end 0.5 -3.396) (width 0.25) (layer "F.Cu") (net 4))
 (segment (start 0 -16.05) (end -10.45 -26.5) (width 0.25) (layer "F.Cu") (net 1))
 (segment (start 0 -3.396) (end 0 -16.05) (width 0.25) (layer "F.Cu") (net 1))
 (segment (start -1 -15.05) (end -1 -3.396) (width 0.25) (layer "F.Cu") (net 2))
 (segment (start -12.45 -26.5) (end -1 -15.05) (width 0.25) (layer "F.Cu") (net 2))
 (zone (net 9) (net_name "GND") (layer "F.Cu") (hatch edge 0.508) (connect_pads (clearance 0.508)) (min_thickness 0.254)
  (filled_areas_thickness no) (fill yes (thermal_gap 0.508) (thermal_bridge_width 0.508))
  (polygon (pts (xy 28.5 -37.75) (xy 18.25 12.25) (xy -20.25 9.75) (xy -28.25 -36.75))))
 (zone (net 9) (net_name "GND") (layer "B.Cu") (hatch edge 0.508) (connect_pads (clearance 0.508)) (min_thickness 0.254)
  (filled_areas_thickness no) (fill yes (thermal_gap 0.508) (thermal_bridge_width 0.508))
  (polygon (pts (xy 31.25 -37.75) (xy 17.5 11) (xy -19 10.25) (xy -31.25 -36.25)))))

